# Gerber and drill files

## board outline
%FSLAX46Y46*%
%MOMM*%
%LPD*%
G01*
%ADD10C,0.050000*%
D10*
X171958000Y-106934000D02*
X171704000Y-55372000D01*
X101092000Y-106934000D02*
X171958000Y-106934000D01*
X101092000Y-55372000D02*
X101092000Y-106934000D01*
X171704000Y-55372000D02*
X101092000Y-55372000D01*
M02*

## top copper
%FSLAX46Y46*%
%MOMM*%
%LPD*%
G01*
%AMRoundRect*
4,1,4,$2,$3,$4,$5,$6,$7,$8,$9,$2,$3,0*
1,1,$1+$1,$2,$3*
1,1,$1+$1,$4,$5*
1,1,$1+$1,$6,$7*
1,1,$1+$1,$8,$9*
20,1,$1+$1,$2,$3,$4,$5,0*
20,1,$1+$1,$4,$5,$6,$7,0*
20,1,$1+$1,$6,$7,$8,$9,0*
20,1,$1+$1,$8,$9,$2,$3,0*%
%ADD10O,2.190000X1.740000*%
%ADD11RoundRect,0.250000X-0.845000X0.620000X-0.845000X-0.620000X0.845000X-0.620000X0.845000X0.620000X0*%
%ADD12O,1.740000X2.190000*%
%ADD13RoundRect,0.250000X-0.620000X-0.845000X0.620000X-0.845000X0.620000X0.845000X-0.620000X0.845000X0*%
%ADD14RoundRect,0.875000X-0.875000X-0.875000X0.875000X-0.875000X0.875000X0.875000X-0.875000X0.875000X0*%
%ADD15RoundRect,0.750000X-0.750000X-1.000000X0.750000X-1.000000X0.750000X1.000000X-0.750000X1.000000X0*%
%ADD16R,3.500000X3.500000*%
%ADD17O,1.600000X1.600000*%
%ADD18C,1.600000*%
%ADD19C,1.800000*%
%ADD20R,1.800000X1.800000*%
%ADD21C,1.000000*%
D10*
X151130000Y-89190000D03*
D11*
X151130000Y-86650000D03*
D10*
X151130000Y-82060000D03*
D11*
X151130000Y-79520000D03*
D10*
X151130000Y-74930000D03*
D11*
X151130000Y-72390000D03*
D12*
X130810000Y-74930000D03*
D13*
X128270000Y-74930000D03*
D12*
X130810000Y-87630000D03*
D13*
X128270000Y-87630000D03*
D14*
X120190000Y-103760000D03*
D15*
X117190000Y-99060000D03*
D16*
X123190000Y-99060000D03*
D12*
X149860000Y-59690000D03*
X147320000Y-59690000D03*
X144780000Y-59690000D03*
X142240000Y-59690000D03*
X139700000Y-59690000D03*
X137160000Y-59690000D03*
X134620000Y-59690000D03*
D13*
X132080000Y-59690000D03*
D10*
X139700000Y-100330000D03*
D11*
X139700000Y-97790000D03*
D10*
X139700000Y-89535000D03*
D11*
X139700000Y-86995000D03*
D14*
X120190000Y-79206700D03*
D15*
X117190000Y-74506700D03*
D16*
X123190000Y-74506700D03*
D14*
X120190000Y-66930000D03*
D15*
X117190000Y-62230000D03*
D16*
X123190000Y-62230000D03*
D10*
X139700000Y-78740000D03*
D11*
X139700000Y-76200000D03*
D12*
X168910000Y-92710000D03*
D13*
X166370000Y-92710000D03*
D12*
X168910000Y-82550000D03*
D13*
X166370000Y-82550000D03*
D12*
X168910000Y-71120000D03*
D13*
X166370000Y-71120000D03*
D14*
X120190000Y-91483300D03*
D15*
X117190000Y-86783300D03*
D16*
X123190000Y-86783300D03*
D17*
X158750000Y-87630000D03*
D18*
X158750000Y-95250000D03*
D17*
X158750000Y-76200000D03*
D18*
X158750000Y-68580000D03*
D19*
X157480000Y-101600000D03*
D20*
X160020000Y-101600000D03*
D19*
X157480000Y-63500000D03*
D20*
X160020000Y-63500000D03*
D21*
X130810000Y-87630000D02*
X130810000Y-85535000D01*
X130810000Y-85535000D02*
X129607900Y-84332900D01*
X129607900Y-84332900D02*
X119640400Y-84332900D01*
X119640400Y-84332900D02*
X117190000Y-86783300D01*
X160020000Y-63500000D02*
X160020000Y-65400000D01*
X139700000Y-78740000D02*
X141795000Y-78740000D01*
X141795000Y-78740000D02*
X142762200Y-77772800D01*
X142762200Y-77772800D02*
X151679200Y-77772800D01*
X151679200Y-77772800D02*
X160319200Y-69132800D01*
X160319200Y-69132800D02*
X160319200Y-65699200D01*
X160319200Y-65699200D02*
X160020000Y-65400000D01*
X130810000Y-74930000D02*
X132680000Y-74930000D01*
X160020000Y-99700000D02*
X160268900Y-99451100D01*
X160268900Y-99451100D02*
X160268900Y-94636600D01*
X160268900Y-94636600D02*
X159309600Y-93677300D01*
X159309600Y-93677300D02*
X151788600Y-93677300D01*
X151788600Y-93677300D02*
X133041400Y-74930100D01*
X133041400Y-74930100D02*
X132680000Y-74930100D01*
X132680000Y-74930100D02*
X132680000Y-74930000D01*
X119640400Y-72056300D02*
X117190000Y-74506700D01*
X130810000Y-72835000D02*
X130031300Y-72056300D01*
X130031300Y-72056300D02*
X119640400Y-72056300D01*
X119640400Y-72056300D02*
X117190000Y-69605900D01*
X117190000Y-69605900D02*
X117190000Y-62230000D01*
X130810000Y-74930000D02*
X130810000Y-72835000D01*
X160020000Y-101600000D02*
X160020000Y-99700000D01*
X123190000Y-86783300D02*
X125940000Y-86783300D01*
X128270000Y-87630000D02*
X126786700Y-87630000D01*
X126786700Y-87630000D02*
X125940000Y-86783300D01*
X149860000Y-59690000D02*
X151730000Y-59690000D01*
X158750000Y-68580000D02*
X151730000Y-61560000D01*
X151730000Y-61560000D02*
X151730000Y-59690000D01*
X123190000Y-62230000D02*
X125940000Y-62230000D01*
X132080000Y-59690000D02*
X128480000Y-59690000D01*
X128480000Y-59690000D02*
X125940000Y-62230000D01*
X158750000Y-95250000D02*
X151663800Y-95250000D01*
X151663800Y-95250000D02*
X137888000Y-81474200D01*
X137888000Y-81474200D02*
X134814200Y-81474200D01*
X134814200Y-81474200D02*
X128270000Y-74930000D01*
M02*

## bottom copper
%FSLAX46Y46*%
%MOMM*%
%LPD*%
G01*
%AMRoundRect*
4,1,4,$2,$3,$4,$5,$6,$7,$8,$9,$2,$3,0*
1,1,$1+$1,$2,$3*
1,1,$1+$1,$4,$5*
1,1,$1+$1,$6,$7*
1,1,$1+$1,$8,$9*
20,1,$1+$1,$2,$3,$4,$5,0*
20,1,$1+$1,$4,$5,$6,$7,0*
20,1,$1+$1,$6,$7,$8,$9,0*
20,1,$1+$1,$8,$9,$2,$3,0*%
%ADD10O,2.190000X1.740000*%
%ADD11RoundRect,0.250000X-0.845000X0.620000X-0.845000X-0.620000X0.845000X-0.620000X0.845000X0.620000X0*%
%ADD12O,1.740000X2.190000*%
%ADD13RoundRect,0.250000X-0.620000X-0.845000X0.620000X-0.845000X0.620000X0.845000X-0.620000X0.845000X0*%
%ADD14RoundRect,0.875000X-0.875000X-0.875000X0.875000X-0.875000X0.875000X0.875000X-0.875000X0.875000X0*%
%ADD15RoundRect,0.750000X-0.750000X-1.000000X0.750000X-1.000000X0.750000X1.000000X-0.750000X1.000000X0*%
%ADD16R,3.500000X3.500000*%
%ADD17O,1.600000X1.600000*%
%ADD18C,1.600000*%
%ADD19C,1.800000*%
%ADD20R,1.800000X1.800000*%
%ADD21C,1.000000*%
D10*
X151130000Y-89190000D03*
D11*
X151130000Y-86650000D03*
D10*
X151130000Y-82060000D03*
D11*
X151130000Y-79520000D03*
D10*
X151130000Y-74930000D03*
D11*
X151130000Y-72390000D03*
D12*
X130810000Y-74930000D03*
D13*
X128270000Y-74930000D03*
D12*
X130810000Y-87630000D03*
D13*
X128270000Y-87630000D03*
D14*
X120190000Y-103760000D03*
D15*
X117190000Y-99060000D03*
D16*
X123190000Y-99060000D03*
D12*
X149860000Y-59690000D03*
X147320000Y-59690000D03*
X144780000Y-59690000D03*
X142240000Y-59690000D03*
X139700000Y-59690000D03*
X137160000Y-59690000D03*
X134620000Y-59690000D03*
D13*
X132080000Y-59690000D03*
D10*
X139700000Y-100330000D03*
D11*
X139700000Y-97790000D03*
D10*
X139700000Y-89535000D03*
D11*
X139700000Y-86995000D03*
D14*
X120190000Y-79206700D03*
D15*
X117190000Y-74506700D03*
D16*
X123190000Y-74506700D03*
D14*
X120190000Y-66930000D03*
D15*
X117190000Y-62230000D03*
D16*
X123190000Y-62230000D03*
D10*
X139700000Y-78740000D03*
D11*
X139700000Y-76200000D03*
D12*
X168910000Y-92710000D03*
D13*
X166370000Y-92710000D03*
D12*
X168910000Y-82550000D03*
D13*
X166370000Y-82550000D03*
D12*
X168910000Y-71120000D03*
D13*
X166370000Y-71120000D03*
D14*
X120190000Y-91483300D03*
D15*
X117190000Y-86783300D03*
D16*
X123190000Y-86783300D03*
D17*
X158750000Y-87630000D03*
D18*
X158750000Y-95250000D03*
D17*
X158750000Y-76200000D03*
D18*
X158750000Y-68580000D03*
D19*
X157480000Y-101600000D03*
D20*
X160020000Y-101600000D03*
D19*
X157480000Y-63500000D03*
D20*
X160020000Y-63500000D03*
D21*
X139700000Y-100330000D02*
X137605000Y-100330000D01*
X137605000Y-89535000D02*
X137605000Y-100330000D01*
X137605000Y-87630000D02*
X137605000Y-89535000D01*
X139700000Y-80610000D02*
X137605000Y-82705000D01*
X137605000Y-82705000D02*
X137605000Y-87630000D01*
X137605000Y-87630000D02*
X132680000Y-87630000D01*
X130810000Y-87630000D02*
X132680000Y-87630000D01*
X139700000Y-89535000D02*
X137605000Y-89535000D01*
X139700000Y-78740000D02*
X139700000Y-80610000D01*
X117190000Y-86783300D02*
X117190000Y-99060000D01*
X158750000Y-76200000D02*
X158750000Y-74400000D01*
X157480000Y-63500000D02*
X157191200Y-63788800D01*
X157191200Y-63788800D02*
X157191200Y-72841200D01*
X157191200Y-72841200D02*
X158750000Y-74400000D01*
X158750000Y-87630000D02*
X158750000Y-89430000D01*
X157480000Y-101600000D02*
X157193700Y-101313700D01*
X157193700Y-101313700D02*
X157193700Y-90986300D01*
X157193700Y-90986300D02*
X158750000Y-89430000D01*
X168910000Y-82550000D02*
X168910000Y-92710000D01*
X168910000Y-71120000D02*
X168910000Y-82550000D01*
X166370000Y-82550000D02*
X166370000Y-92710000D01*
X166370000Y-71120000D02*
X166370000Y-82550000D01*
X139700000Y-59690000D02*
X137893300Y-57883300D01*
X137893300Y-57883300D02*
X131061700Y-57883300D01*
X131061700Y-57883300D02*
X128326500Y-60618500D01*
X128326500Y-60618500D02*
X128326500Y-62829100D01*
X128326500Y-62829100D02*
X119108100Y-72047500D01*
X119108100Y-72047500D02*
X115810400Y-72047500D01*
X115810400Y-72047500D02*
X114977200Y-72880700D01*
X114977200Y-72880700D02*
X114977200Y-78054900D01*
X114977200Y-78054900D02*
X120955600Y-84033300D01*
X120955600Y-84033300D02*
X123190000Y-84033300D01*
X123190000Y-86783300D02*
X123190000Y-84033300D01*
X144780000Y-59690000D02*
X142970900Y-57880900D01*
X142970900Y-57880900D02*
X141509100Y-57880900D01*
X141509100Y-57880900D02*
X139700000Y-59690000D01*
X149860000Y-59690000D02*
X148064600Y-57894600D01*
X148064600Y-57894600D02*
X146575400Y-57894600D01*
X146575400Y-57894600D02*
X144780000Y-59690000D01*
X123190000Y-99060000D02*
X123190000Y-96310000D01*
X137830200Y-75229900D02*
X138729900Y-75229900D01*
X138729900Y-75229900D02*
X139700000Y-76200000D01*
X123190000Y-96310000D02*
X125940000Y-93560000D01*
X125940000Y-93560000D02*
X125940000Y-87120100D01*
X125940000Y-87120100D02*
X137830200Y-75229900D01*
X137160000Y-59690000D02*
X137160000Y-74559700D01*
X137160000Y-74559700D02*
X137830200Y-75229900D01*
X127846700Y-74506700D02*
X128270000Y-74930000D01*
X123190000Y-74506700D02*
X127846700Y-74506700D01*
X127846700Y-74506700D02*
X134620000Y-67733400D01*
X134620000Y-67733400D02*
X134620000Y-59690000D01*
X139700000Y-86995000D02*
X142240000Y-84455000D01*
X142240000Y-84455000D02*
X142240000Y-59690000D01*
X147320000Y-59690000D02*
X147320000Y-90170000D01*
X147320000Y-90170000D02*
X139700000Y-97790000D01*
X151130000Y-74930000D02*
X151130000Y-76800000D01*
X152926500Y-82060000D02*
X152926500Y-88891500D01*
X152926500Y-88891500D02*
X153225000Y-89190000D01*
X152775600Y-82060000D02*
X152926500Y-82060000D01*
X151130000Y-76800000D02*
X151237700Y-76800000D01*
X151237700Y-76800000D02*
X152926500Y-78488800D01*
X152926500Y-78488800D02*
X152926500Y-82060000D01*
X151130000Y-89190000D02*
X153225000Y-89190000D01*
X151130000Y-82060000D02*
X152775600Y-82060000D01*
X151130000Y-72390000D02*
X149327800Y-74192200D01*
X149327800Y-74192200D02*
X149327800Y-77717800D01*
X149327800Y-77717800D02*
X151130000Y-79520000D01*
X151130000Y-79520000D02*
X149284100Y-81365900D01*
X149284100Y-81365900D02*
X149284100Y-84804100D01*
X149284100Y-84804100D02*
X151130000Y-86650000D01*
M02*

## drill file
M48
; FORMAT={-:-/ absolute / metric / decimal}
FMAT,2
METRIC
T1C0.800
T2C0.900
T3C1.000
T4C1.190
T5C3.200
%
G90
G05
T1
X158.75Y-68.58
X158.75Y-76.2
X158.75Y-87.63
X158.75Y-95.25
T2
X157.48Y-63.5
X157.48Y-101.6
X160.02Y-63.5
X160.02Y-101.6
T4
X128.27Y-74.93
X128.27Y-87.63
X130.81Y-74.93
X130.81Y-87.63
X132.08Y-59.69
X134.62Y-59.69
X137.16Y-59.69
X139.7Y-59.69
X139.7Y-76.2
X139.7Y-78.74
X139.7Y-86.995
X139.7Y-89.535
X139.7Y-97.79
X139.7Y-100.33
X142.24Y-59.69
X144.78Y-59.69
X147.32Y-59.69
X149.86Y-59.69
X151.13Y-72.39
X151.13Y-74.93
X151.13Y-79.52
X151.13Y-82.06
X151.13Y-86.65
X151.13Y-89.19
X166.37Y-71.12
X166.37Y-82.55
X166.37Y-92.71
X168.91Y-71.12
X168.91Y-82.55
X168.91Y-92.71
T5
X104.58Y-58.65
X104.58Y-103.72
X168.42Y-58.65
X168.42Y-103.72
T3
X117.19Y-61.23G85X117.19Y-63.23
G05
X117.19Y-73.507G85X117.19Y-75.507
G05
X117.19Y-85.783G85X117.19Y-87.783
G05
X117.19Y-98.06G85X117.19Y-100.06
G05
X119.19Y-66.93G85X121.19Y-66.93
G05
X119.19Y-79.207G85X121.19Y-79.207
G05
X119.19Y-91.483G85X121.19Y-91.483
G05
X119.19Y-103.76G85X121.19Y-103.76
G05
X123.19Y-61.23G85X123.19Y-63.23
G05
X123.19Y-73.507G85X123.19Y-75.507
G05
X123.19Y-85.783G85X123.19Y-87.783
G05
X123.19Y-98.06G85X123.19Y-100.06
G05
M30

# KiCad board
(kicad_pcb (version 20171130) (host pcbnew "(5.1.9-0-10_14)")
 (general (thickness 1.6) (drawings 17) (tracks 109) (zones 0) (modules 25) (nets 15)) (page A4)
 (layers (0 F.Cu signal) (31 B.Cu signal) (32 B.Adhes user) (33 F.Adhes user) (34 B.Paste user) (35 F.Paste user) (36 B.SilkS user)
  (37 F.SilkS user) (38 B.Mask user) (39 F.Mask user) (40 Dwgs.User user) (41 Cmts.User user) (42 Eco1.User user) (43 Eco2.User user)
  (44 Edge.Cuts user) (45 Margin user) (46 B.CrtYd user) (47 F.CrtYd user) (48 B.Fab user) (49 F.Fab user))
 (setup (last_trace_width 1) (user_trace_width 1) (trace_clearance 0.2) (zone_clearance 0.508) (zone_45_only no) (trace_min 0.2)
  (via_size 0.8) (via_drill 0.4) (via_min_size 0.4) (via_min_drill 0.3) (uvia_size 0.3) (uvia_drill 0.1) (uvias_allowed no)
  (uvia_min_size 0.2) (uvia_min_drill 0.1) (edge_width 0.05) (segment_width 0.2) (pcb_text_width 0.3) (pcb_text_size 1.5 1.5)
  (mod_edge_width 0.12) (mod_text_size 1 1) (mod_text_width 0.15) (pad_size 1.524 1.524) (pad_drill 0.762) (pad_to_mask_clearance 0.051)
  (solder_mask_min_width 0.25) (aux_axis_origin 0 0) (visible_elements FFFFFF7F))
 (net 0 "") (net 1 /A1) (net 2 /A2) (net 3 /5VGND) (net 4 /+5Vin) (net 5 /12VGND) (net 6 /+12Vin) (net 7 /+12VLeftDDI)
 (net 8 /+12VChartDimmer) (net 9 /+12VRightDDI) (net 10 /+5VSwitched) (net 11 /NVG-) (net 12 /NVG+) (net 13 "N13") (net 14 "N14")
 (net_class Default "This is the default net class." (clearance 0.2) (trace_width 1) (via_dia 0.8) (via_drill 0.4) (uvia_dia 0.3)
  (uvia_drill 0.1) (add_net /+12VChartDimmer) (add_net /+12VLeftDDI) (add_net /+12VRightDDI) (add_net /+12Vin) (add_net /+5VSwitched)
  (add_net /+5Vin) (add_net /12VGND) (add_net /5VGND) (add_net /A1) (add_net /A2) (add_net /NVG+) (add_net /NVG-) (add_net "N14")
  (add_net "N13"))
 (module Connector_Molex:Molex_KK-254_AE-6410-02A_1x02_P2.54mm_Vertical (layer F.Cu) (at 151.13 86.65 270)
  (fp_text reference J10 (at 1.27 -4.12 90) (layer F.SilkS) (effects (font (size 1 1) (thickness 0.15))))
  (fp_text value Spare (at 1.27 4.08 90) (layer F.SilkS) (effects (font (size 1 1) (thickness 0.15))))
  (pad 2 thru_hole oval (at 2.54 0 270) (size 1.74 2.19) (drill 1.19) (layers *.Cu *.Mask) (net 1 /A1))
  (pad 1 thru_hole roundrect (at 0 0 270) (size 1.74 2.19) (drill 1.19) (layers *.Cu *.Mask) (roundrect_rratio 0.143678) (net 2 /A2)))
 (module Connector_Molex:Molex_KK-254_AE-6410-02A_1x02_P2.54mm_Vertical (layer F.Cu) (at 151.13 79.52 270)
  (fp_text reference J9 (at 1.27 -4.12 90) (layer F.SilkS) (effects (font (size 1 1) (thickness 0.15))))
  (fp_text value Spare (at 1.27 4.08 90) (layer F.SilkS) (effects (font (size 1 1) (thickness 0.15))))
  (pad 2 thru_hole oval (at 2.54 0 270) (size 1.74 2.19) (drill 1.19) (layers *.Cu *.Mask) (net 1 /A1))
  (pad 1 thru_hole roundrect (at 0 0 270) (size 1.74 2.19) (drill 1.19) (layers *.Cu *.Mask) (roundrect_rratio 0.143678) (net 2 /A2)))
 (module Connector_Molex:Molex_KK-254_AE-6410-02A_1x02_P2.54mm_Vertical (layer F.Cu) (at 151.13 72.39 270)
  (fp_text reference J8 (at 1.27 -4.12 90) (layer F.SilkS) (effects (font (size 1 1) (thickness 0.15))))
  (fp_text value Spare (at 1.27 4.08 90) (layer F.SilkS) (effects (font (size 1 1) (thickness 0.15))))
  (pad 2 thru_hole oval (at 2.54 0 270) (size 1.74 2.19) (drill 1.19) (layers *.Cu *.Mask) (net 1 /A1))
  (pad 1 thru_hole roundrect (at 0 0 270) (size 1.74 2.19) (drill 1.19) (layers *.Cu *.Mask) (roundrect_rratio 0.143678) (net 2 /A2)))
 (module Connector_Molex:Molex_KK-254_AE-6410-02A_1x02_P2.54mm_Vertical (layer F.Cu) (at 128.27 74.93)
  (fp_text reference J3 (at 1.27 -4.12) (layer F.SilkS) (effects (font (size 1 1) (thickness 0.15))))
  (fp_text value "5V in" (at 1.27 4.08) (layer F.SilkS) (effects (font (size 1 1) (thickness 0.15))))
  (pad 2 thru_hole oval (at 2.54 0) (size 1.74 2.19) (drill 1.19) (layers *.Cu *.Mask) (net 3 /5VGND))
  (pad 1 thru_hole roundrect (at 0 0) (size 1.74 2.19) (drill 1.19) (layers *.Cu *.Mask) (roundrect_rratio 0.143678) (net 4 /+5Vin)))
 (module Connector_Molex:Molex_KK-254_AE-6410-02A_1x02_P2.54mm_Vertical (layer F.Cu) (at 128.27 87.63)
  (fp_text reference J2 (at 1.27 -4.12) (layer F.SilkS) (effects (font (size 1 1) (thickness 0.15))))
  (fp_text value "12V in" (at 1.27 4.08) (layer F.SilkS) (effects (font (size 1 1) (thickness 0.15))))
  (pad 2 thru_hole oval (at 2.54 0) (size 1.74 2.19) (drill 1.19) (layers *.Cu *.Mask) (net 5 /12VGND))
  (pad 1 thru_hole roundrect (at 0 0) (size 1.74 2.19) (drill 1.19) (layers *.Cu *.Mask) (roundrect_rratio 0.143678) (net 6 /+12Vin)))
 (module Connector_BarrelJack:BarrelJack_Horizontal (layer F.Cu) (at 123.19 99.06)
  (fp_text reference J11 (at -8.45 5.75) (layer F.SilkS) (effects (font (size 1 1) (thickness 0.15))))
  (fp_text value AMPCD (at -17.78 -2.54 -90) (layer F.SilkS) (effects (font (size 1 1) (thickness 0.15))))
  (pad 3 thru_hole roundrect (at -3 4.7) (size 3.5 3.5) (drill oval 3 1) (layers *.Cu *.Mask) (roundrect_rratio 0.25))
  (pad 2 thru_hole roundrect (at -6 0) (size 3 3.5) (drill oval 1 3) (layers *.Cu *.Mask) (roundrect_rratio 0.25) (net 5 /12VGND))
  (pad 1 thru_hole rect (at 0 0) (size 3.5 3.5) (drill oval 1 3) (layers *.Cu *.Mask) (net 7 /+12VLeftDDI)))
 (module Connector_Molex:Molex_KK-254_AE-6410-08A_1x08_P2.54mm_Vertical (layer F.Cu) (at 132.08 59.69)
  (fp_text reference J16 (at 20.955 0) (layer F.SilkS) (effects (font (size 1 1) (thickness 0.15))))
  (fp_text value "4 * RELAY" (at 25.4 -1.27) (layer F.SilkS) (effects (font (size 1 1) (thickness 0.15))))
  (pad 8 thru_hole oval (at 17.78 0) (size 1.74 2.19) (drill 1.19) (layers *.Cu *.Mask) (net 6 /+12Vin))
  (pad 7 thru_hole oval (at 15.24 0) (size 1.74 2.19) (drill 1.19) (layers *.Cu *.Mask) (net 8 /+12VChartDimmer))
  (pad 6 thru_hole oval (at 12.7 0) (size 1.74 2.19) (drill 1.19) (layers *.Cu *.Mask) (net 6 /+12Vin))
  (pad 5 thru_hole oval (at 10.16 0) (size 1.74 2.19) (drill 1.19) (layers *.Cu *.Mask) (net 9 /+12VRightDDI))
  (pad 4 thru_hole oval (at 7.62 0) (size 1.74 2.19) (drill 1.19) (layers *.Cu *.Mask) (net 6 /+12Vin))
  (pad 3 thru_hole oval (at 5.08 0) (size 1.74 2.19) (drill 1.19) (layers *.Cu *.Mask) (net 7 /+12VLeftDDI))
  (pad 2 thru_hole oval (at 2.54 0) (size 1.74 2.19) (drill 1.19) (layers *.Cu *.Mask) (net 4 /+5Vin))
  (pad 1 thru_hole roundrect (at 0 0) (size 1.74 2.19) (drill 1.19) (layers *.Cu *.Mask) (roundrect_rratio 0.143678) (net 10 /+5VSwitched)))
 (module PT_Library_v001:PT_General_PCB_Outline (layer F.Cu) (at 137.006 80.5581)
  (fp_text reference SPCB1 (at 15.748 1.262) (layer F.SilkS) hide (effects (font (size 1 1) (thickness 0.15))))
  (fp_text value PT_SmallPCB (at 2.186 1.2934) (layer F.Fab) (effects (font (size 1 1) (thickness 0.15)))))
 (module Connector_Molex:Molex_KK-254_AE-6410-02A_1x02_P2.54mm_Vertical (layer F.Cu) (at 139.7 97.79 270)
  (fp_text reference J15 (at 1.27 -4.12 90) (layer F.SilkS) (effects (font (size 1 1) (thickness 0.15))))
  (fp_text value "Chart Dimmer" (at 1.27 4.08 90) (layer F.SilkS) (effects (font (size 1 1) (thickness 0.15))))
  (pad 2 thru_hole oval (at 2.54 0 270) (size 1.74 2.19) (drill 1.19) (layers *.Cu *.Mask) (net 5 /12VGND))
  (pad 1 thru_hole roundrect (at 0 0 270) (size 1.74 2.19) (drill 1.19) (layers *.Cu *.Mask) (roundrect_rratio 0.143678)
   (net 8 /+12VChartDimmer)))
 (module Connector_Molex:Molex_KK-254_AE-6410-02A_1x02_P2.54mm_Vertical (layer F.Cu) (at 139.7 86.995 270)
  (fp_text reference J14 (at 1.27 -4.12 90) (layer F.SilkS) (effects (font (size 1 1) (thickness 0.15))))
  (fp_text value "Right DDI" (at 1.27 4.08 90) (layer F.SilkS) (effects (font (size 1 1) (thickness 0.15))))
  (pad 2 thru_hole oval (at 2.54 0 270) (size 1.74 2.19) (drill 1.19) (layers *.Cu *.Mask) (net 5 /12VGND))
  (pad 1 thru_hole roundrect (at 0 0 270) (size 1.74 2.19) (drill 1.19) (layers *.Cu *.Mask) (roundrect_rratio 0.143678)
   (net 9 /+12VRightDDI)))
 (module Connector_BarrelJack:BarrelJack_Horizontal (layer F.Cu) (at 123.19 74.5067)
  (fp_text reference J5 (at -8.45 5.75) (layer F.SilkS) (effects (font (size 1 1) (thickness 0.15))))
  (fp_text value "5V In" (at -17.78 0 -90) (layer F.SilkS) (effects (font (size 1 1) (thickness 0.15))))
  (pad 3 thru_hole roundrect (at -3 4.7) (size 3.5 3.5) (drill oval 3 1) (layers *.Cu *.Mask) (roundrect_rratio 0.25))
  (pad 2 thru_hole roundrect (at -6 0) (size 3 3.5) (drill oval 1 3) (layers *.Cu *.Mask) (roundrect_rratio 0.25) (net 3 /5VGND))
  (pad 1 thru_hole rect (at 0 0) (size 3.5 3.5) (drill oval 1 3) (layers *.Cu *.Mask) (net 4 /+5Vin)))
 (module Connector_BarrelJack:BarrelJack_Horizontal (layer F.Cu) (at 123.19 62.23)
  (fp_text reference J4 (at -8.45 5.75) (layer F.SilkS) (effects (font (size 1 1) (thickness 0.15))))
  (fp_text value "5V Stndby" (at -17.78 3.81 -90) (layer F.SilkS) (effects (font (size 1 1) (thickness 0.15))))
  (pad 3 thru_hole roundrect (at -3 4.7) (size 3.5 3.5) (drill oval 3 1) (layers *.Cu *.Mask) (roundrect_rratio 0.25))
  (pad 2 thru_hole roundrect (at -6 0) (size 3 3.5) (drill oval 1 3) (layers *.Cu *.Mask) (roundrect_rratio 0.25) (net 3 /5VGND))
  (pad 1 thru_hole rect (at 0 0) (size 3.5 3.5) (drill oval 1 3) (layers *.Cu *.Mask) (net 10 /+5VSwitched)))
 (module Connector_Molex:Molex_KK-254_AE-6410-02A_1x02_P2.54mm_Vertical (layer F.Cu) (at 139.7 76.2 270)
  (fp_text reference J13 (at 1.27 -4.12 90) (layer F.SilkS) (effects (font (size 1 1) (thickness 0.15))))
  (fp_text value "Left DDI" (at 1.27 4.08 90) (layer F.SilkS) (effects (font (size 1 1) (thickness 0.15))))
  (pad 2 thru_hole oval (at 2.54 0 270) (size 1.74 2.19) (drill 1.19) (layers *.Cu *.Mask) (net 5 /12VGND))
  (pad 1 thru_hole roundrect (at 0 0 270) (size 1.74 2.19) (drill 1.19) (layers *.Cu *.Mask) (roundrect_rratio 0.143678)
   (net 7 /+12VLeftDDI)))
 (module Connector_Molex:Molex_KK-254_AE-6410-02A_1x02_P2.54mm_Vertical (layer F.Cu) (at 166.37 92.71)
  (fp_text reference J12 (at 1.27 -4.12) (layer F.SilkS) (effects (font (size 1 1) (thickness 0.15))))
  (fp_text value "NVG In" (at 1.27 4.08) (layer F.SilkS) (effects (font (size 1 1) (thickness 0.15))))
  (pad 2 thru_hole oval (at 2.54 0) (size 1.74 2.19) (drill 1.19) (layers *.Cu *.Mask) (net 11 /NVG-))
  (pad 1 thru_hole roundrect (at 0 0) (size 1.74 2.19) (drill 1.19) (layers *.Cu *.Mask) (roundrect_rratio 0.143678) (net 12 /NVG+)))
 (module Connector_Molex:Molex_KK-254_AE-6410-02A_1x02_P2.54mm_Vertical (layer F.Cu) (at 166.37 82.55)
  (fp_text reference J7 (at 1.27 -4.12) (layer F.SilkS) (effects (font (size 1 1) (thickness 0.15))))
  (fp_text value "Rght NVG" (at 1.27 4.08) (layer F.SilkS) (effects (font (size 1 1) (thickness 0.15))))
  (pad 2 thru_hole oval (at 2.54 0) (size 1.74 2.19) (drill 1.19) (layers *.Cu *.Mask) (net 11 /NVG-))
  (pad 1 thru_hole roundrect (at 0 0) (size 1.74 2.19) (drill 1.19) (layers *.Cu *.Mask) (roundrect_rratio 0.143678) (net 12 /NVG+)))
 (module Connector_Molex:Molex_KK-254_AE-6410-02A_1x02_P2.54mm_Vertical (layer F.Cu) (at 166.37 71.12)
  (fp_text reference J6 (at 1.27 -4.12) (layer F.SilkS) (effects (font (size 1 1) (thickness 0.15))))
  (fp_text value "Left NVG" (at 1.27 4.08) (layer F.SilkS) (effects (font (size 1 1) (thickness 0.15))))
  (pad 2 thru_hole oval (at 2.54 0) (size 1.74 2.19) (drill 1.19) (layers *.Cu *.Mask) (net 11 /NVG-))
  (pad 1 thru_hole roundrect (at 0 0) (size 1.74 2.19) (drill 1.19) (layers *.Cu *.Mask) (roundrect_rratio 0.143678) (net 12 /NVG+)))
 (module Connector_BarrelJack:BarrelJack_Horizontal (layer F.Cu) (at 123.19 86.7833)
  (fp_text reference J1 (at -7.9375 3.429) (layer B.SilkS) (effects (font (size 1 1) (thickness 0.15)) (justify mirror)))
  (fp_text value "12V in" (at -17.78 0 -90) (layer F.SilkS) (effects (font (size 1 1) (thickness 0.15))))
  (pad 3 thru_hole roundrect (at -3 4.7) (size 3.5 3.5) (drill oval 3 1) (layers *.Cu *.Mask) (roundrect_rratio 0.25))
  (pad 2 thru_hole roundrect (at -6 0) (size 3 3.5) (drill oval 1 3) (layers *.Cu *.Mask) (roundrect_rratio 0.25) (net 5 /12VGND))
  (pad 1 thru_hole rect (at 0 0) (size 3.5 3.5) (drill oval 1 3) (layers *.Cu *.Mask) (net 6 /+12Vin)))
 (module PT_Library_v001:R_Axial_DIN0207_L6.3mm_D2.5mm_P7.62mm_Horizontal (layer F.Cu) (at 158.75 95.25 90)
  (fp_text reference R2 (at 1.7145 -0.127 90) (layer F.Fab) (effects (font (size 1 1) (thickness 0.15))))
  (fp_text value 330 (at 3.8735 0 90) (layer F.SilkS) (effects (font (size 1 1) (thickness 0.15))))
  (pad 2 thru_hole oval (at 7.62 0 90) (size 1.6 1.6) (drill 0.8) (layers *.Cu *.Mask) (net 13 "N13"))
  (pad 1 thru_hole circle (at 0 0 90) (size 1.6 1.6) (drill 0.8) (layers *.Cu *.Mask) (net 4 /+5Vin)))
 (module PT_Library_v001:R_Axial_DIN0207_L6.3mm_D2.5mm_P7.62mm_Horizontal (layer F.Cu) (at 158.75 68.58 270)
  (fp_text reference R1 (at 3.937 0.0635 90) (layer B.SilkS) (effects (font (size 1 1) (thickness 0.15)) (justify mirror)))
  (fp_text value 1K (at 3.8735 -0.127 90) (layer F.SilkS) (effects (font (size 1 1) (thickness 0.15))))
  (pad 2 thru_hole oval (at 7.62 0 270) (size 1.6 1.6) (drill 0.8) (layers *.Cu *.Mask) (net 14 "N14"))
  (pad 1 thru_hole circle (at 0 0 270) (size 1.6 1.6) (drill 0.8) (layers *.Cu *.Mask) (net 6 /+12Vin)))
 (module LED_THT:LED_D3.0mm (layer F.Cu) (at 160.02 101.6 180)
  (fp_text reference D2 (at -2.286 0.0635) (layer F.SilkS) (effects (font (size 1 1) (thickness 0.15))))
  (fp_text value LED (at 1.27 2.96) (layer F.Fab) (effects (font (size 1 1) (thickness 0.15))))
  (pad 2 thru_hole circle (at 2.54 0 180) (size 1.8 1.8) (drill 0.9) (layers *.Cu *.Mask) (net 13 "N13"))
  (pad 1 thru_hole rect (at 0 0 180) (size 1.8 1.8) (drill 0.9) (layers *.Cu *.Mask) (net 3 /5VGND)))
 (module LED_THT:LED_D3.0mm (layer F.Cu) (at 160.02 63.5 180)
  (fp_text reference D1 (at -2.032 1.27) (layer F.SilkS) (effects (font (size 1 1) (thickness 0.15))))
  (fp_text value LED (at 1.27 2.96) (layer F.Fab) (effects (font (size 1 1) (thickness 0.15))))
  (pad 2 thru_hole circle (at 2.54 0 180) (size 1.8 1.8) (drill 0.9) (layers *.Cu *.Mask) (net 14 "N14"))
  (pad 1 thru_hole rect (at 0 0 180) (size 1.8 1.8) (drill 0.9) (layers *.Cu *.Mask) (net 5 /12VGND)))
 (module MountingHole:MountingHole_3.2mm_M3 (layer F.Cu) (at 168.42 103.72)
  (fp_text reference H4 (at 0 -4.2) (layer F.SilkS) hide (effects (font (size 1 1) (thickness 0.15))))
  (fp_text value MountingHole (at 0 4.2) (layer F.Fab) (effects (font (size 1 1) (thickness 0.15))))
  (pad 1 np_thru_hole circle (at 0 0) (size 3.2 3.2) (drill 3.2) (layers *.Cu *.Mask)))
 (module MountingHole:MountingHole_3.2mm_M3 (layer F.Cu) (at 168.42 58.65)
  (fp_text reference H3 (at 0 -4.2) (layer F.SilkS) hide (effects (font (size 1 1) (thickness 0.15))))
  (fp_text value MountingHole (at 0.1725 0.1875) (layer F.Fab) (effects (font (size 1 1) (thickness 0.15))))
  (pad 1 np_thru_hole circle (at 0 0) (size 3.2 3.2) (drill 3.2) (layers *.Cu *.Mask)))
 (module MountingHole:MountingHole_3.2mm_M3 (layer F.Cu) (at 104.58 103.72)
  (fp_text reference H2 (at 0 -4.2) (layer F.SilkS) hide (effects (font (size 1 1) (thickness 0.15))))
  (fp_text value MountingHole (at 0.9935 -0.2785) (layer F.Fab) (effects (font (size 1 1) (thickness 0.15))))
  (pad 1 np_thru_hole circle (at 0 0) (size 3.2 3.2) (drill 3.2) (layers *.Cu *.Mask)))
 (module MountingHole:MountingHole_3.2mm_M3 (layer F.Cu) (at 104.58 58.65)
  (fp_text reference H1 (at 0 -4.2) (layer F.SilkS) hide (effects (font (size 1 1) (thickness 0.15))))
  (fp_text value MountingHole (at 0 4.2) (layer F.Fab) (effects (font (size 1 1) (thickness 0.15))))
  (pad 1 np_thru_hole circle (at 0 0) (size 3.2 3.2) (drill 3.2) (layers *.Cu *.Mask)))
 (gr_line (start 171.958 106.934) (end 171.704 55.372) (layer Edge.Cuts) (width 0.05))
 (gr_line (start 101.092 106.934) (end 171.958 106.934) (layer Edge.Cuts) (width 0.05))
 (gr_line (start 101.092 55.372) (end 101.092 106.934) (layer Edge.Cuts) (width 0.05))
 (gr_line (start 171.704 55.372) (end 101.092 55.372) (layer Edge.Cuts) (width 0.05))
 (segment (start 130.81 87.63) (end 130.81 85.535) (width 1) (layer F.Cu) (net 5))
 (segment (start 130.81 85.535) (end 129.6079 84.3329) (width 1) (layer F.Cu) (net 5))
 (segment (start 129.6079 84.3329) (end 119.6404 84.3329) (width 1) (layer F.Cu) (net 5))
 (segment (start 119.6404 84.3329) (end 117.19 86.7833) (width 1) (layer F.Cu) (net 5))
 (segment (start 139.7 100.33) (end 137.605 100.33) (width 1) (layer B.Cu) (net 5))
 (segment (start 137.605 89.535) (end 137.605 100.33) (width 1) (layer B.Cu) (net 5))
 (segment (start 137.605 87.63) (end 137.605 89.535) (width 1) (layer B.Cu) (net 5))
 (segment (start 139.7 80.61) (end 137.605 82.705) (width 1) (layer B.Cu) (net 5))
 (segment (start 137.605 82.705) (end 137.605 87.63) (width 1) (layer B.Cu) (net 5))
 (segment (start 137.605 87.63) (end 132.68 87.63) (width 1) (layer B.Cu) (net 5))
 (segment (start 130.81 87.63) (end 132.68 87.63) (width 1) (layer B.Cu) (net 5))
 (segment (start 139.7 89.535) (end 137.605 89.535) (width 1) (layer B.Cu) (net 5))
 (segment (start 139.7 78.74) (end 139.7 80.61) (width 1) (layer B.Cu) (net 5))
 (segment (start 160.02 63.5) (end 160.02 65.4) (width 1) (layer F.Cu) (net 5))
 (segment (start 139.7 78.74) (end 141.795 78.74) (width 1) (layer F.Cu) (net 5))
 (segment (start 141.795 78.74) (end 142.7622 77.7728) (width 1) (layer F.Cu) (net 5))
 (segment (start 142.7622 77.7728) (end 151.6792 77.7728) (width 1) (layer F.Cu) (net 5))
 (segment (start 151.6792 77.7728) (end 160.3192 69.1328) (width 1) (layer F.Cu) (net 5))
 (segment (start 160.3192 69.1328) (end 160.3192 65.6992) (width 1) (layer F.Cu) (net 5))
 (segment (start 160.3192 65.6992) (end 160.02 65.4) (width 1) (layer F.Cu) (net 5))
 (segment (start 117.19 86.7833) (end 117.19 99.06) (width 1) (layer B.Cu) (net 5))
 (segment (start 130.81 74.93) (end 132.68 74.93) (width 1) (layer F.Cu) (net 3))
 (segment (start 160.02 99.7) (end 160.2689 99.4511) (width 1) (layer F.Cu) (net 3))
 (segment (start 160.2689 99.4511) (end 160.2689 94.6366) (width 1) (layer F.Cu) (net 3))
 (segment (start 160.2689 94.6366) (end 159.3096 93.6773) (width 1) (layer F.Cu) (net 3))
 (segment (start 159.3096 93.6773) (end 151.7886 93.6773) (width 1) (layer F.Cu) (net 3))
 (segment (start 151.7886 93.6773) (end 133.0414 74.9301) (width 1) (layer F.Cu) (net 3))
 (segment (start 133.0414 74.9301) (end 132.68 74.9301) (width 1) (layer F.Cu) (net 3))
 (segment (start 132.68 74.9301) (end 132.68 74.93) (width 1) (layer F.Cu) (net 3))
 (segment (start 119.6404 72.0563) (end 117.19 74.5067) (width 1) (layer F.Cu) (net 3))
 (segment (start 130.81 72.835) (end 130.0313 72.0563) (width 1) (layer F.Cu) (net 3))
 (segment (start 130.0313 72.0563) (end 119.6404 72.0563) (width 1) (layer F.Cu) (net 3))
 (segment (start 119.6404 72.0563) (end 117.19 69.6059) (width 1) (layer F.Cu) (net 3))
 (segment (start 117.19 69.6059) (end 117.19 62.23) (width 1) (layer F.Cu) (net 3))
 (segment (start 130.81 74.93) (end 130.81 72.835) (width 1) (layer F.Cu) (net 3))
 (segment (start 160.02 101.6) (end 160.02 99.7) (width 1) (layer F.Cu) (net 3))
 (segment (start 158.75 76.2) (end 158.75 74.4) (width 1) (layer B.Cu) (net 14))
 (segment (start 157.48 63.5) (end 157.1912 63.7888) (width 1) (layer B.Cu) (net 14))
 (segment (start 157.1912 63.7888) (end 157.1912 72.8412) (width 1) (layer B.Cu) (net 14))
 (segment (start 157.1912 72.8412) (end 158.75 74.4) (width 1) (layer B.Cu) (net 14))
 (segment (start 158.75 87.63) (end 158.75 89.43) (width 1) (layer B.Cu) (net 13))
 (segment (start 157.48 101.6) (end 157.1937 101.3137) (width 1) (layer B.Cu) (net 13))
 (segment (start 157.1937 101.3137) (end 157.1937 90.9863) (width 1) (layer B.Cu) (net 13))
 (segment (start 157.1937 90.9863) (end 158.75 89.43) (width 1) (layer B.Cu) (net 13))
 (segment (start 168.91 82.55) (end 168.91 92.71) (width 1) (layer B.Cu) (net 11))
 (segment (start 168.91 71.12) (end 168.91 82.55) (width 1) (layer B.Cu) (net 11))
 (segment (start 166.37 82.55) (end 166.37 92.71) (width 1) (layer B.Cu) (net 12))
 (segment (start 166.37 71.12) (end 166.37 82.55) (width 1) (layer B.Cu) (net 12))
 (segment (start 139.7 59.69) (end 137.8933 57.8833) (width 1) (layer B.Cu) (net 6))
 (segment (start 137.8933 57.8833) (end 131.0617 57.8833) (width 1) (layer B.Cu) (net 6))
 (segment (start 131.0617 57.8833) (end 128.3265 60.6185) (width 1) (layer B.Cu) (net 6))
 (segment (start 128.3265 60.6185) (end 128.3265 62.8291) (width 1) (layer B.Cu) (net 6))
 (segment (start 128.3265 62.8291) (end 119.1081 72.0475) (width 1) (layer B.Cu) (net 6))
 (segment (start 119.1081 72.0475) (end 115.8104 72.0475) (width 1) (layer B.Cu) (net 6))
 (segment (start 115.8104 72.0475) (end 114.9772 72.8807) (width 1) (layer B.Cu) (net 6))
 (segment (start 114.9772 72.8807) (end 114.9772 78.0549) (width 1) (layer B.Cu) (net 6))
 (segment (start 114.9772 78.0549) (end 120.9556 84.0333) (width 1) (layer B.Cu) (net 6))
 (segment (start 120.9556 84.0333) (end 123.19 84.0333) (width 1) (layer B.Cu) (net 6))
 (segment (start 123.19 86.7833) (end 123.19 84.0333) (width 1) (layer B.Cu) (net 6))
 (segment (start 144.78 59.69) (end 142.9709 57.8809) (width 1) (layer B.Cu) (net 6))
 (segment (start 142.9709 57.8809) (end 141.5091 57.8809) (width 1) (layer B.Cu) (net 6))
 (segment (start 141.5091 57.8809) (end 139.7 59.69) (width 1) (layer B.Cu) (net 6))
 (segment (start 149.86 59.69) (end 148.0646 57.8946) (width 1) (layer B.Cu) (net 6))
 (segment (start 148.0646 57.8946) (end 146.5754 57.8946) (width 1) (layer B.Cu) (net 6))
 (segment (start 146.5754 57.8946) (end 144.78 59.69) (width 1) (layer B.Cu) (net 6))
 (segment (start 123.19 86.7833) (end 125.94 86.7833) (width 1) (layer F.Cu) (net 6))
 (segment (start 128.27 87.63) (end 126.7867 87.63) (width 1) (layer F.Cu) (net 6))
 (segment (start 126.7867 87.63) (end 125.94 86.7833) (width 1) (layer F.Cu) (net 6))
 (segment (start 149.86 59.69) (end 151.73 59.69) (width 1) (layer F.Cu) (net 6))
 (segment (start 158.75 68.58) (end 151.73 61.56) (width 1) (layer F.Cu) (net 6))
 (segment (start 151.73 61.56) (end 151.73 59.69) (width 1) (layer F.Cu) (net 6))
 (segment (start 123.19 99.06) (end 123.19 96.31) (width 1) (layer B.Cu) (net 7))
 (segment (start 137.8302 75.2299) (end 138.7299 75.2299) (width 1) (layer B.Cu) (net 7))
 (segment (start 138.7299 75.2299) (end 139.7 76.2) (width 1) (layer B.Cu) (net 7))
 (segment (start 123.19 96.31) (end 125.94 93.56) (width 1) (layer B.Cu) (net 7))
 (segment (start 125.94 93.56) (end 125.94 87.1201) (width 1) (layer B.Cu) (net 7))
 (segment (start 125.94 87.1201) (end 137.8302 75.2299) (width 1) (layer B.Cu) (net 7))
 (segment (start 137.16 59.69) (end 137.16 74.5597) (width 1) (layer B.Cu) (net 7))
 (segment (start 137.16 74.5597) (end 137.8302 75.2299) (width 1) (layer B.Cu) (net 7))
 (segment (start 123.19 62.23) (end 125.94 62.23) (width 1) (layer F.Cu) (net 10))
 (segment (start 132.08 59.69) (end 128.48 59.69) (width 1) (layer F.Cu) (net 10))
 (segment (start 128.48 59.69) (end 125.94 62.23) (width 1) (layer F.Cu) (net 10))
 (segment (start 158.75 95.25) (end 151.6638 95.25) (width 1) (layer F.Cu) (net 4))
 (segment (start 151.6638 95.25) (end 137.888 81.4742) (width 1) (layer F.Cu) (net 4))
 (segment (start 137.888 81.4742) (end 134.8142 81.4742) (width 1) (layer F.Cu) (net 4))
 (segment (start 134.8142 81.4742) (end 128.27 74.93) (width 1) (layer F.Cu) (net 4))
 (segment (start 127.8467 74.5067) (end 128.27 74.93) (width 1) (layer B.Cu) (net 4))
 (segment (start 123.19 74.5067) (end 127.8467 74.5067) (width 1) (layer B.Cu) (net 4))
 (segment (start 127.8467 74.5067) (end 134.62 67.7334) (width 1) (layer B.Cu) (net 4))
 (segment (start 134.62 67.7334) (end 134.62 59.69) (width 1) (layer B.Cu) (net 4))
 (segment (start 139.7 86.995) (end 142.24 84.455) (width 1) (layer B.Cu) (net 9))
 (segment (start 142.24 84.455) (end 142.24 59.69) (width 1) (layer B.Cu) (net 9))
 (segment (start 147.32 59.69) (end 147.32 90.17) (width 1) (layer B.Cu) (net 8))
 (segment (start 147.32 90.17) (end 139.7 97.79) (width 1) (layer B.Cu) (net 8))
 (segment (start 151.13 74.93) (end 151.13 76.8) (width 1) (layer B.Cu) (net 1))
 (segment (start 152.9265 82.06) (end 152.9265 88.8915) (width 1) (layer B.Cu) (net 1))
 (segment (start 152.9265 88.8915) (end 153.225 89.19) (width 1) (layer B.Cu) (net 1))
 (segment (start 152.7756 82.06) (end 152.9265 82.06) (width 1) (layer B.Cu) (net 1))
 (segment (start 151.13 76.8) (end 151.2377 76.8) (width 1) (layer B.Cu) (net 1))
 (segment (start 151.2377 76.8) (end 152.9265 78.4888) (width 1) (layer B.Cu) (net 1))
 (segment (start 152.9265 78.4888) (end 152.9265 82.06) (width 1) (layer B.Cu) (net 1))
 (segment (start 151.13 89.19) (end 153.225 89.19) (width 1) (layer B.Cu) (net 1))
 (segment (start 151.13 82.06) (end 152.7756 82.06) (width 1) (layer B.Cu) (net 1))
 (segment (start 151.13 72.39) (end 149.3278 74.1922) (width 1) (layer B.Cu) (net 2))
 (segment (start 149.3278 74.1922) (end 149.3278 77.7178) (width 1) (layer B.Cu) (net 2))
 (segment (start 149.3278 77.7178) (end 151.13 79.52) (width 1) (layer B.Cu) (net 2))
 (segment (start 151.13 79.52) (end 149.2841 81.3659) (width 1) (layer B.Cu) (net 2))
 (segment (start 149.2841 81.3659) (end 149.2841 84.8041) (width 1) (layer B.Cu) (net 2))
 (segment (start 149.2841 84.8041) (end 151.13 86.65) (width 1) (layer B.Cu) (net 2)))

